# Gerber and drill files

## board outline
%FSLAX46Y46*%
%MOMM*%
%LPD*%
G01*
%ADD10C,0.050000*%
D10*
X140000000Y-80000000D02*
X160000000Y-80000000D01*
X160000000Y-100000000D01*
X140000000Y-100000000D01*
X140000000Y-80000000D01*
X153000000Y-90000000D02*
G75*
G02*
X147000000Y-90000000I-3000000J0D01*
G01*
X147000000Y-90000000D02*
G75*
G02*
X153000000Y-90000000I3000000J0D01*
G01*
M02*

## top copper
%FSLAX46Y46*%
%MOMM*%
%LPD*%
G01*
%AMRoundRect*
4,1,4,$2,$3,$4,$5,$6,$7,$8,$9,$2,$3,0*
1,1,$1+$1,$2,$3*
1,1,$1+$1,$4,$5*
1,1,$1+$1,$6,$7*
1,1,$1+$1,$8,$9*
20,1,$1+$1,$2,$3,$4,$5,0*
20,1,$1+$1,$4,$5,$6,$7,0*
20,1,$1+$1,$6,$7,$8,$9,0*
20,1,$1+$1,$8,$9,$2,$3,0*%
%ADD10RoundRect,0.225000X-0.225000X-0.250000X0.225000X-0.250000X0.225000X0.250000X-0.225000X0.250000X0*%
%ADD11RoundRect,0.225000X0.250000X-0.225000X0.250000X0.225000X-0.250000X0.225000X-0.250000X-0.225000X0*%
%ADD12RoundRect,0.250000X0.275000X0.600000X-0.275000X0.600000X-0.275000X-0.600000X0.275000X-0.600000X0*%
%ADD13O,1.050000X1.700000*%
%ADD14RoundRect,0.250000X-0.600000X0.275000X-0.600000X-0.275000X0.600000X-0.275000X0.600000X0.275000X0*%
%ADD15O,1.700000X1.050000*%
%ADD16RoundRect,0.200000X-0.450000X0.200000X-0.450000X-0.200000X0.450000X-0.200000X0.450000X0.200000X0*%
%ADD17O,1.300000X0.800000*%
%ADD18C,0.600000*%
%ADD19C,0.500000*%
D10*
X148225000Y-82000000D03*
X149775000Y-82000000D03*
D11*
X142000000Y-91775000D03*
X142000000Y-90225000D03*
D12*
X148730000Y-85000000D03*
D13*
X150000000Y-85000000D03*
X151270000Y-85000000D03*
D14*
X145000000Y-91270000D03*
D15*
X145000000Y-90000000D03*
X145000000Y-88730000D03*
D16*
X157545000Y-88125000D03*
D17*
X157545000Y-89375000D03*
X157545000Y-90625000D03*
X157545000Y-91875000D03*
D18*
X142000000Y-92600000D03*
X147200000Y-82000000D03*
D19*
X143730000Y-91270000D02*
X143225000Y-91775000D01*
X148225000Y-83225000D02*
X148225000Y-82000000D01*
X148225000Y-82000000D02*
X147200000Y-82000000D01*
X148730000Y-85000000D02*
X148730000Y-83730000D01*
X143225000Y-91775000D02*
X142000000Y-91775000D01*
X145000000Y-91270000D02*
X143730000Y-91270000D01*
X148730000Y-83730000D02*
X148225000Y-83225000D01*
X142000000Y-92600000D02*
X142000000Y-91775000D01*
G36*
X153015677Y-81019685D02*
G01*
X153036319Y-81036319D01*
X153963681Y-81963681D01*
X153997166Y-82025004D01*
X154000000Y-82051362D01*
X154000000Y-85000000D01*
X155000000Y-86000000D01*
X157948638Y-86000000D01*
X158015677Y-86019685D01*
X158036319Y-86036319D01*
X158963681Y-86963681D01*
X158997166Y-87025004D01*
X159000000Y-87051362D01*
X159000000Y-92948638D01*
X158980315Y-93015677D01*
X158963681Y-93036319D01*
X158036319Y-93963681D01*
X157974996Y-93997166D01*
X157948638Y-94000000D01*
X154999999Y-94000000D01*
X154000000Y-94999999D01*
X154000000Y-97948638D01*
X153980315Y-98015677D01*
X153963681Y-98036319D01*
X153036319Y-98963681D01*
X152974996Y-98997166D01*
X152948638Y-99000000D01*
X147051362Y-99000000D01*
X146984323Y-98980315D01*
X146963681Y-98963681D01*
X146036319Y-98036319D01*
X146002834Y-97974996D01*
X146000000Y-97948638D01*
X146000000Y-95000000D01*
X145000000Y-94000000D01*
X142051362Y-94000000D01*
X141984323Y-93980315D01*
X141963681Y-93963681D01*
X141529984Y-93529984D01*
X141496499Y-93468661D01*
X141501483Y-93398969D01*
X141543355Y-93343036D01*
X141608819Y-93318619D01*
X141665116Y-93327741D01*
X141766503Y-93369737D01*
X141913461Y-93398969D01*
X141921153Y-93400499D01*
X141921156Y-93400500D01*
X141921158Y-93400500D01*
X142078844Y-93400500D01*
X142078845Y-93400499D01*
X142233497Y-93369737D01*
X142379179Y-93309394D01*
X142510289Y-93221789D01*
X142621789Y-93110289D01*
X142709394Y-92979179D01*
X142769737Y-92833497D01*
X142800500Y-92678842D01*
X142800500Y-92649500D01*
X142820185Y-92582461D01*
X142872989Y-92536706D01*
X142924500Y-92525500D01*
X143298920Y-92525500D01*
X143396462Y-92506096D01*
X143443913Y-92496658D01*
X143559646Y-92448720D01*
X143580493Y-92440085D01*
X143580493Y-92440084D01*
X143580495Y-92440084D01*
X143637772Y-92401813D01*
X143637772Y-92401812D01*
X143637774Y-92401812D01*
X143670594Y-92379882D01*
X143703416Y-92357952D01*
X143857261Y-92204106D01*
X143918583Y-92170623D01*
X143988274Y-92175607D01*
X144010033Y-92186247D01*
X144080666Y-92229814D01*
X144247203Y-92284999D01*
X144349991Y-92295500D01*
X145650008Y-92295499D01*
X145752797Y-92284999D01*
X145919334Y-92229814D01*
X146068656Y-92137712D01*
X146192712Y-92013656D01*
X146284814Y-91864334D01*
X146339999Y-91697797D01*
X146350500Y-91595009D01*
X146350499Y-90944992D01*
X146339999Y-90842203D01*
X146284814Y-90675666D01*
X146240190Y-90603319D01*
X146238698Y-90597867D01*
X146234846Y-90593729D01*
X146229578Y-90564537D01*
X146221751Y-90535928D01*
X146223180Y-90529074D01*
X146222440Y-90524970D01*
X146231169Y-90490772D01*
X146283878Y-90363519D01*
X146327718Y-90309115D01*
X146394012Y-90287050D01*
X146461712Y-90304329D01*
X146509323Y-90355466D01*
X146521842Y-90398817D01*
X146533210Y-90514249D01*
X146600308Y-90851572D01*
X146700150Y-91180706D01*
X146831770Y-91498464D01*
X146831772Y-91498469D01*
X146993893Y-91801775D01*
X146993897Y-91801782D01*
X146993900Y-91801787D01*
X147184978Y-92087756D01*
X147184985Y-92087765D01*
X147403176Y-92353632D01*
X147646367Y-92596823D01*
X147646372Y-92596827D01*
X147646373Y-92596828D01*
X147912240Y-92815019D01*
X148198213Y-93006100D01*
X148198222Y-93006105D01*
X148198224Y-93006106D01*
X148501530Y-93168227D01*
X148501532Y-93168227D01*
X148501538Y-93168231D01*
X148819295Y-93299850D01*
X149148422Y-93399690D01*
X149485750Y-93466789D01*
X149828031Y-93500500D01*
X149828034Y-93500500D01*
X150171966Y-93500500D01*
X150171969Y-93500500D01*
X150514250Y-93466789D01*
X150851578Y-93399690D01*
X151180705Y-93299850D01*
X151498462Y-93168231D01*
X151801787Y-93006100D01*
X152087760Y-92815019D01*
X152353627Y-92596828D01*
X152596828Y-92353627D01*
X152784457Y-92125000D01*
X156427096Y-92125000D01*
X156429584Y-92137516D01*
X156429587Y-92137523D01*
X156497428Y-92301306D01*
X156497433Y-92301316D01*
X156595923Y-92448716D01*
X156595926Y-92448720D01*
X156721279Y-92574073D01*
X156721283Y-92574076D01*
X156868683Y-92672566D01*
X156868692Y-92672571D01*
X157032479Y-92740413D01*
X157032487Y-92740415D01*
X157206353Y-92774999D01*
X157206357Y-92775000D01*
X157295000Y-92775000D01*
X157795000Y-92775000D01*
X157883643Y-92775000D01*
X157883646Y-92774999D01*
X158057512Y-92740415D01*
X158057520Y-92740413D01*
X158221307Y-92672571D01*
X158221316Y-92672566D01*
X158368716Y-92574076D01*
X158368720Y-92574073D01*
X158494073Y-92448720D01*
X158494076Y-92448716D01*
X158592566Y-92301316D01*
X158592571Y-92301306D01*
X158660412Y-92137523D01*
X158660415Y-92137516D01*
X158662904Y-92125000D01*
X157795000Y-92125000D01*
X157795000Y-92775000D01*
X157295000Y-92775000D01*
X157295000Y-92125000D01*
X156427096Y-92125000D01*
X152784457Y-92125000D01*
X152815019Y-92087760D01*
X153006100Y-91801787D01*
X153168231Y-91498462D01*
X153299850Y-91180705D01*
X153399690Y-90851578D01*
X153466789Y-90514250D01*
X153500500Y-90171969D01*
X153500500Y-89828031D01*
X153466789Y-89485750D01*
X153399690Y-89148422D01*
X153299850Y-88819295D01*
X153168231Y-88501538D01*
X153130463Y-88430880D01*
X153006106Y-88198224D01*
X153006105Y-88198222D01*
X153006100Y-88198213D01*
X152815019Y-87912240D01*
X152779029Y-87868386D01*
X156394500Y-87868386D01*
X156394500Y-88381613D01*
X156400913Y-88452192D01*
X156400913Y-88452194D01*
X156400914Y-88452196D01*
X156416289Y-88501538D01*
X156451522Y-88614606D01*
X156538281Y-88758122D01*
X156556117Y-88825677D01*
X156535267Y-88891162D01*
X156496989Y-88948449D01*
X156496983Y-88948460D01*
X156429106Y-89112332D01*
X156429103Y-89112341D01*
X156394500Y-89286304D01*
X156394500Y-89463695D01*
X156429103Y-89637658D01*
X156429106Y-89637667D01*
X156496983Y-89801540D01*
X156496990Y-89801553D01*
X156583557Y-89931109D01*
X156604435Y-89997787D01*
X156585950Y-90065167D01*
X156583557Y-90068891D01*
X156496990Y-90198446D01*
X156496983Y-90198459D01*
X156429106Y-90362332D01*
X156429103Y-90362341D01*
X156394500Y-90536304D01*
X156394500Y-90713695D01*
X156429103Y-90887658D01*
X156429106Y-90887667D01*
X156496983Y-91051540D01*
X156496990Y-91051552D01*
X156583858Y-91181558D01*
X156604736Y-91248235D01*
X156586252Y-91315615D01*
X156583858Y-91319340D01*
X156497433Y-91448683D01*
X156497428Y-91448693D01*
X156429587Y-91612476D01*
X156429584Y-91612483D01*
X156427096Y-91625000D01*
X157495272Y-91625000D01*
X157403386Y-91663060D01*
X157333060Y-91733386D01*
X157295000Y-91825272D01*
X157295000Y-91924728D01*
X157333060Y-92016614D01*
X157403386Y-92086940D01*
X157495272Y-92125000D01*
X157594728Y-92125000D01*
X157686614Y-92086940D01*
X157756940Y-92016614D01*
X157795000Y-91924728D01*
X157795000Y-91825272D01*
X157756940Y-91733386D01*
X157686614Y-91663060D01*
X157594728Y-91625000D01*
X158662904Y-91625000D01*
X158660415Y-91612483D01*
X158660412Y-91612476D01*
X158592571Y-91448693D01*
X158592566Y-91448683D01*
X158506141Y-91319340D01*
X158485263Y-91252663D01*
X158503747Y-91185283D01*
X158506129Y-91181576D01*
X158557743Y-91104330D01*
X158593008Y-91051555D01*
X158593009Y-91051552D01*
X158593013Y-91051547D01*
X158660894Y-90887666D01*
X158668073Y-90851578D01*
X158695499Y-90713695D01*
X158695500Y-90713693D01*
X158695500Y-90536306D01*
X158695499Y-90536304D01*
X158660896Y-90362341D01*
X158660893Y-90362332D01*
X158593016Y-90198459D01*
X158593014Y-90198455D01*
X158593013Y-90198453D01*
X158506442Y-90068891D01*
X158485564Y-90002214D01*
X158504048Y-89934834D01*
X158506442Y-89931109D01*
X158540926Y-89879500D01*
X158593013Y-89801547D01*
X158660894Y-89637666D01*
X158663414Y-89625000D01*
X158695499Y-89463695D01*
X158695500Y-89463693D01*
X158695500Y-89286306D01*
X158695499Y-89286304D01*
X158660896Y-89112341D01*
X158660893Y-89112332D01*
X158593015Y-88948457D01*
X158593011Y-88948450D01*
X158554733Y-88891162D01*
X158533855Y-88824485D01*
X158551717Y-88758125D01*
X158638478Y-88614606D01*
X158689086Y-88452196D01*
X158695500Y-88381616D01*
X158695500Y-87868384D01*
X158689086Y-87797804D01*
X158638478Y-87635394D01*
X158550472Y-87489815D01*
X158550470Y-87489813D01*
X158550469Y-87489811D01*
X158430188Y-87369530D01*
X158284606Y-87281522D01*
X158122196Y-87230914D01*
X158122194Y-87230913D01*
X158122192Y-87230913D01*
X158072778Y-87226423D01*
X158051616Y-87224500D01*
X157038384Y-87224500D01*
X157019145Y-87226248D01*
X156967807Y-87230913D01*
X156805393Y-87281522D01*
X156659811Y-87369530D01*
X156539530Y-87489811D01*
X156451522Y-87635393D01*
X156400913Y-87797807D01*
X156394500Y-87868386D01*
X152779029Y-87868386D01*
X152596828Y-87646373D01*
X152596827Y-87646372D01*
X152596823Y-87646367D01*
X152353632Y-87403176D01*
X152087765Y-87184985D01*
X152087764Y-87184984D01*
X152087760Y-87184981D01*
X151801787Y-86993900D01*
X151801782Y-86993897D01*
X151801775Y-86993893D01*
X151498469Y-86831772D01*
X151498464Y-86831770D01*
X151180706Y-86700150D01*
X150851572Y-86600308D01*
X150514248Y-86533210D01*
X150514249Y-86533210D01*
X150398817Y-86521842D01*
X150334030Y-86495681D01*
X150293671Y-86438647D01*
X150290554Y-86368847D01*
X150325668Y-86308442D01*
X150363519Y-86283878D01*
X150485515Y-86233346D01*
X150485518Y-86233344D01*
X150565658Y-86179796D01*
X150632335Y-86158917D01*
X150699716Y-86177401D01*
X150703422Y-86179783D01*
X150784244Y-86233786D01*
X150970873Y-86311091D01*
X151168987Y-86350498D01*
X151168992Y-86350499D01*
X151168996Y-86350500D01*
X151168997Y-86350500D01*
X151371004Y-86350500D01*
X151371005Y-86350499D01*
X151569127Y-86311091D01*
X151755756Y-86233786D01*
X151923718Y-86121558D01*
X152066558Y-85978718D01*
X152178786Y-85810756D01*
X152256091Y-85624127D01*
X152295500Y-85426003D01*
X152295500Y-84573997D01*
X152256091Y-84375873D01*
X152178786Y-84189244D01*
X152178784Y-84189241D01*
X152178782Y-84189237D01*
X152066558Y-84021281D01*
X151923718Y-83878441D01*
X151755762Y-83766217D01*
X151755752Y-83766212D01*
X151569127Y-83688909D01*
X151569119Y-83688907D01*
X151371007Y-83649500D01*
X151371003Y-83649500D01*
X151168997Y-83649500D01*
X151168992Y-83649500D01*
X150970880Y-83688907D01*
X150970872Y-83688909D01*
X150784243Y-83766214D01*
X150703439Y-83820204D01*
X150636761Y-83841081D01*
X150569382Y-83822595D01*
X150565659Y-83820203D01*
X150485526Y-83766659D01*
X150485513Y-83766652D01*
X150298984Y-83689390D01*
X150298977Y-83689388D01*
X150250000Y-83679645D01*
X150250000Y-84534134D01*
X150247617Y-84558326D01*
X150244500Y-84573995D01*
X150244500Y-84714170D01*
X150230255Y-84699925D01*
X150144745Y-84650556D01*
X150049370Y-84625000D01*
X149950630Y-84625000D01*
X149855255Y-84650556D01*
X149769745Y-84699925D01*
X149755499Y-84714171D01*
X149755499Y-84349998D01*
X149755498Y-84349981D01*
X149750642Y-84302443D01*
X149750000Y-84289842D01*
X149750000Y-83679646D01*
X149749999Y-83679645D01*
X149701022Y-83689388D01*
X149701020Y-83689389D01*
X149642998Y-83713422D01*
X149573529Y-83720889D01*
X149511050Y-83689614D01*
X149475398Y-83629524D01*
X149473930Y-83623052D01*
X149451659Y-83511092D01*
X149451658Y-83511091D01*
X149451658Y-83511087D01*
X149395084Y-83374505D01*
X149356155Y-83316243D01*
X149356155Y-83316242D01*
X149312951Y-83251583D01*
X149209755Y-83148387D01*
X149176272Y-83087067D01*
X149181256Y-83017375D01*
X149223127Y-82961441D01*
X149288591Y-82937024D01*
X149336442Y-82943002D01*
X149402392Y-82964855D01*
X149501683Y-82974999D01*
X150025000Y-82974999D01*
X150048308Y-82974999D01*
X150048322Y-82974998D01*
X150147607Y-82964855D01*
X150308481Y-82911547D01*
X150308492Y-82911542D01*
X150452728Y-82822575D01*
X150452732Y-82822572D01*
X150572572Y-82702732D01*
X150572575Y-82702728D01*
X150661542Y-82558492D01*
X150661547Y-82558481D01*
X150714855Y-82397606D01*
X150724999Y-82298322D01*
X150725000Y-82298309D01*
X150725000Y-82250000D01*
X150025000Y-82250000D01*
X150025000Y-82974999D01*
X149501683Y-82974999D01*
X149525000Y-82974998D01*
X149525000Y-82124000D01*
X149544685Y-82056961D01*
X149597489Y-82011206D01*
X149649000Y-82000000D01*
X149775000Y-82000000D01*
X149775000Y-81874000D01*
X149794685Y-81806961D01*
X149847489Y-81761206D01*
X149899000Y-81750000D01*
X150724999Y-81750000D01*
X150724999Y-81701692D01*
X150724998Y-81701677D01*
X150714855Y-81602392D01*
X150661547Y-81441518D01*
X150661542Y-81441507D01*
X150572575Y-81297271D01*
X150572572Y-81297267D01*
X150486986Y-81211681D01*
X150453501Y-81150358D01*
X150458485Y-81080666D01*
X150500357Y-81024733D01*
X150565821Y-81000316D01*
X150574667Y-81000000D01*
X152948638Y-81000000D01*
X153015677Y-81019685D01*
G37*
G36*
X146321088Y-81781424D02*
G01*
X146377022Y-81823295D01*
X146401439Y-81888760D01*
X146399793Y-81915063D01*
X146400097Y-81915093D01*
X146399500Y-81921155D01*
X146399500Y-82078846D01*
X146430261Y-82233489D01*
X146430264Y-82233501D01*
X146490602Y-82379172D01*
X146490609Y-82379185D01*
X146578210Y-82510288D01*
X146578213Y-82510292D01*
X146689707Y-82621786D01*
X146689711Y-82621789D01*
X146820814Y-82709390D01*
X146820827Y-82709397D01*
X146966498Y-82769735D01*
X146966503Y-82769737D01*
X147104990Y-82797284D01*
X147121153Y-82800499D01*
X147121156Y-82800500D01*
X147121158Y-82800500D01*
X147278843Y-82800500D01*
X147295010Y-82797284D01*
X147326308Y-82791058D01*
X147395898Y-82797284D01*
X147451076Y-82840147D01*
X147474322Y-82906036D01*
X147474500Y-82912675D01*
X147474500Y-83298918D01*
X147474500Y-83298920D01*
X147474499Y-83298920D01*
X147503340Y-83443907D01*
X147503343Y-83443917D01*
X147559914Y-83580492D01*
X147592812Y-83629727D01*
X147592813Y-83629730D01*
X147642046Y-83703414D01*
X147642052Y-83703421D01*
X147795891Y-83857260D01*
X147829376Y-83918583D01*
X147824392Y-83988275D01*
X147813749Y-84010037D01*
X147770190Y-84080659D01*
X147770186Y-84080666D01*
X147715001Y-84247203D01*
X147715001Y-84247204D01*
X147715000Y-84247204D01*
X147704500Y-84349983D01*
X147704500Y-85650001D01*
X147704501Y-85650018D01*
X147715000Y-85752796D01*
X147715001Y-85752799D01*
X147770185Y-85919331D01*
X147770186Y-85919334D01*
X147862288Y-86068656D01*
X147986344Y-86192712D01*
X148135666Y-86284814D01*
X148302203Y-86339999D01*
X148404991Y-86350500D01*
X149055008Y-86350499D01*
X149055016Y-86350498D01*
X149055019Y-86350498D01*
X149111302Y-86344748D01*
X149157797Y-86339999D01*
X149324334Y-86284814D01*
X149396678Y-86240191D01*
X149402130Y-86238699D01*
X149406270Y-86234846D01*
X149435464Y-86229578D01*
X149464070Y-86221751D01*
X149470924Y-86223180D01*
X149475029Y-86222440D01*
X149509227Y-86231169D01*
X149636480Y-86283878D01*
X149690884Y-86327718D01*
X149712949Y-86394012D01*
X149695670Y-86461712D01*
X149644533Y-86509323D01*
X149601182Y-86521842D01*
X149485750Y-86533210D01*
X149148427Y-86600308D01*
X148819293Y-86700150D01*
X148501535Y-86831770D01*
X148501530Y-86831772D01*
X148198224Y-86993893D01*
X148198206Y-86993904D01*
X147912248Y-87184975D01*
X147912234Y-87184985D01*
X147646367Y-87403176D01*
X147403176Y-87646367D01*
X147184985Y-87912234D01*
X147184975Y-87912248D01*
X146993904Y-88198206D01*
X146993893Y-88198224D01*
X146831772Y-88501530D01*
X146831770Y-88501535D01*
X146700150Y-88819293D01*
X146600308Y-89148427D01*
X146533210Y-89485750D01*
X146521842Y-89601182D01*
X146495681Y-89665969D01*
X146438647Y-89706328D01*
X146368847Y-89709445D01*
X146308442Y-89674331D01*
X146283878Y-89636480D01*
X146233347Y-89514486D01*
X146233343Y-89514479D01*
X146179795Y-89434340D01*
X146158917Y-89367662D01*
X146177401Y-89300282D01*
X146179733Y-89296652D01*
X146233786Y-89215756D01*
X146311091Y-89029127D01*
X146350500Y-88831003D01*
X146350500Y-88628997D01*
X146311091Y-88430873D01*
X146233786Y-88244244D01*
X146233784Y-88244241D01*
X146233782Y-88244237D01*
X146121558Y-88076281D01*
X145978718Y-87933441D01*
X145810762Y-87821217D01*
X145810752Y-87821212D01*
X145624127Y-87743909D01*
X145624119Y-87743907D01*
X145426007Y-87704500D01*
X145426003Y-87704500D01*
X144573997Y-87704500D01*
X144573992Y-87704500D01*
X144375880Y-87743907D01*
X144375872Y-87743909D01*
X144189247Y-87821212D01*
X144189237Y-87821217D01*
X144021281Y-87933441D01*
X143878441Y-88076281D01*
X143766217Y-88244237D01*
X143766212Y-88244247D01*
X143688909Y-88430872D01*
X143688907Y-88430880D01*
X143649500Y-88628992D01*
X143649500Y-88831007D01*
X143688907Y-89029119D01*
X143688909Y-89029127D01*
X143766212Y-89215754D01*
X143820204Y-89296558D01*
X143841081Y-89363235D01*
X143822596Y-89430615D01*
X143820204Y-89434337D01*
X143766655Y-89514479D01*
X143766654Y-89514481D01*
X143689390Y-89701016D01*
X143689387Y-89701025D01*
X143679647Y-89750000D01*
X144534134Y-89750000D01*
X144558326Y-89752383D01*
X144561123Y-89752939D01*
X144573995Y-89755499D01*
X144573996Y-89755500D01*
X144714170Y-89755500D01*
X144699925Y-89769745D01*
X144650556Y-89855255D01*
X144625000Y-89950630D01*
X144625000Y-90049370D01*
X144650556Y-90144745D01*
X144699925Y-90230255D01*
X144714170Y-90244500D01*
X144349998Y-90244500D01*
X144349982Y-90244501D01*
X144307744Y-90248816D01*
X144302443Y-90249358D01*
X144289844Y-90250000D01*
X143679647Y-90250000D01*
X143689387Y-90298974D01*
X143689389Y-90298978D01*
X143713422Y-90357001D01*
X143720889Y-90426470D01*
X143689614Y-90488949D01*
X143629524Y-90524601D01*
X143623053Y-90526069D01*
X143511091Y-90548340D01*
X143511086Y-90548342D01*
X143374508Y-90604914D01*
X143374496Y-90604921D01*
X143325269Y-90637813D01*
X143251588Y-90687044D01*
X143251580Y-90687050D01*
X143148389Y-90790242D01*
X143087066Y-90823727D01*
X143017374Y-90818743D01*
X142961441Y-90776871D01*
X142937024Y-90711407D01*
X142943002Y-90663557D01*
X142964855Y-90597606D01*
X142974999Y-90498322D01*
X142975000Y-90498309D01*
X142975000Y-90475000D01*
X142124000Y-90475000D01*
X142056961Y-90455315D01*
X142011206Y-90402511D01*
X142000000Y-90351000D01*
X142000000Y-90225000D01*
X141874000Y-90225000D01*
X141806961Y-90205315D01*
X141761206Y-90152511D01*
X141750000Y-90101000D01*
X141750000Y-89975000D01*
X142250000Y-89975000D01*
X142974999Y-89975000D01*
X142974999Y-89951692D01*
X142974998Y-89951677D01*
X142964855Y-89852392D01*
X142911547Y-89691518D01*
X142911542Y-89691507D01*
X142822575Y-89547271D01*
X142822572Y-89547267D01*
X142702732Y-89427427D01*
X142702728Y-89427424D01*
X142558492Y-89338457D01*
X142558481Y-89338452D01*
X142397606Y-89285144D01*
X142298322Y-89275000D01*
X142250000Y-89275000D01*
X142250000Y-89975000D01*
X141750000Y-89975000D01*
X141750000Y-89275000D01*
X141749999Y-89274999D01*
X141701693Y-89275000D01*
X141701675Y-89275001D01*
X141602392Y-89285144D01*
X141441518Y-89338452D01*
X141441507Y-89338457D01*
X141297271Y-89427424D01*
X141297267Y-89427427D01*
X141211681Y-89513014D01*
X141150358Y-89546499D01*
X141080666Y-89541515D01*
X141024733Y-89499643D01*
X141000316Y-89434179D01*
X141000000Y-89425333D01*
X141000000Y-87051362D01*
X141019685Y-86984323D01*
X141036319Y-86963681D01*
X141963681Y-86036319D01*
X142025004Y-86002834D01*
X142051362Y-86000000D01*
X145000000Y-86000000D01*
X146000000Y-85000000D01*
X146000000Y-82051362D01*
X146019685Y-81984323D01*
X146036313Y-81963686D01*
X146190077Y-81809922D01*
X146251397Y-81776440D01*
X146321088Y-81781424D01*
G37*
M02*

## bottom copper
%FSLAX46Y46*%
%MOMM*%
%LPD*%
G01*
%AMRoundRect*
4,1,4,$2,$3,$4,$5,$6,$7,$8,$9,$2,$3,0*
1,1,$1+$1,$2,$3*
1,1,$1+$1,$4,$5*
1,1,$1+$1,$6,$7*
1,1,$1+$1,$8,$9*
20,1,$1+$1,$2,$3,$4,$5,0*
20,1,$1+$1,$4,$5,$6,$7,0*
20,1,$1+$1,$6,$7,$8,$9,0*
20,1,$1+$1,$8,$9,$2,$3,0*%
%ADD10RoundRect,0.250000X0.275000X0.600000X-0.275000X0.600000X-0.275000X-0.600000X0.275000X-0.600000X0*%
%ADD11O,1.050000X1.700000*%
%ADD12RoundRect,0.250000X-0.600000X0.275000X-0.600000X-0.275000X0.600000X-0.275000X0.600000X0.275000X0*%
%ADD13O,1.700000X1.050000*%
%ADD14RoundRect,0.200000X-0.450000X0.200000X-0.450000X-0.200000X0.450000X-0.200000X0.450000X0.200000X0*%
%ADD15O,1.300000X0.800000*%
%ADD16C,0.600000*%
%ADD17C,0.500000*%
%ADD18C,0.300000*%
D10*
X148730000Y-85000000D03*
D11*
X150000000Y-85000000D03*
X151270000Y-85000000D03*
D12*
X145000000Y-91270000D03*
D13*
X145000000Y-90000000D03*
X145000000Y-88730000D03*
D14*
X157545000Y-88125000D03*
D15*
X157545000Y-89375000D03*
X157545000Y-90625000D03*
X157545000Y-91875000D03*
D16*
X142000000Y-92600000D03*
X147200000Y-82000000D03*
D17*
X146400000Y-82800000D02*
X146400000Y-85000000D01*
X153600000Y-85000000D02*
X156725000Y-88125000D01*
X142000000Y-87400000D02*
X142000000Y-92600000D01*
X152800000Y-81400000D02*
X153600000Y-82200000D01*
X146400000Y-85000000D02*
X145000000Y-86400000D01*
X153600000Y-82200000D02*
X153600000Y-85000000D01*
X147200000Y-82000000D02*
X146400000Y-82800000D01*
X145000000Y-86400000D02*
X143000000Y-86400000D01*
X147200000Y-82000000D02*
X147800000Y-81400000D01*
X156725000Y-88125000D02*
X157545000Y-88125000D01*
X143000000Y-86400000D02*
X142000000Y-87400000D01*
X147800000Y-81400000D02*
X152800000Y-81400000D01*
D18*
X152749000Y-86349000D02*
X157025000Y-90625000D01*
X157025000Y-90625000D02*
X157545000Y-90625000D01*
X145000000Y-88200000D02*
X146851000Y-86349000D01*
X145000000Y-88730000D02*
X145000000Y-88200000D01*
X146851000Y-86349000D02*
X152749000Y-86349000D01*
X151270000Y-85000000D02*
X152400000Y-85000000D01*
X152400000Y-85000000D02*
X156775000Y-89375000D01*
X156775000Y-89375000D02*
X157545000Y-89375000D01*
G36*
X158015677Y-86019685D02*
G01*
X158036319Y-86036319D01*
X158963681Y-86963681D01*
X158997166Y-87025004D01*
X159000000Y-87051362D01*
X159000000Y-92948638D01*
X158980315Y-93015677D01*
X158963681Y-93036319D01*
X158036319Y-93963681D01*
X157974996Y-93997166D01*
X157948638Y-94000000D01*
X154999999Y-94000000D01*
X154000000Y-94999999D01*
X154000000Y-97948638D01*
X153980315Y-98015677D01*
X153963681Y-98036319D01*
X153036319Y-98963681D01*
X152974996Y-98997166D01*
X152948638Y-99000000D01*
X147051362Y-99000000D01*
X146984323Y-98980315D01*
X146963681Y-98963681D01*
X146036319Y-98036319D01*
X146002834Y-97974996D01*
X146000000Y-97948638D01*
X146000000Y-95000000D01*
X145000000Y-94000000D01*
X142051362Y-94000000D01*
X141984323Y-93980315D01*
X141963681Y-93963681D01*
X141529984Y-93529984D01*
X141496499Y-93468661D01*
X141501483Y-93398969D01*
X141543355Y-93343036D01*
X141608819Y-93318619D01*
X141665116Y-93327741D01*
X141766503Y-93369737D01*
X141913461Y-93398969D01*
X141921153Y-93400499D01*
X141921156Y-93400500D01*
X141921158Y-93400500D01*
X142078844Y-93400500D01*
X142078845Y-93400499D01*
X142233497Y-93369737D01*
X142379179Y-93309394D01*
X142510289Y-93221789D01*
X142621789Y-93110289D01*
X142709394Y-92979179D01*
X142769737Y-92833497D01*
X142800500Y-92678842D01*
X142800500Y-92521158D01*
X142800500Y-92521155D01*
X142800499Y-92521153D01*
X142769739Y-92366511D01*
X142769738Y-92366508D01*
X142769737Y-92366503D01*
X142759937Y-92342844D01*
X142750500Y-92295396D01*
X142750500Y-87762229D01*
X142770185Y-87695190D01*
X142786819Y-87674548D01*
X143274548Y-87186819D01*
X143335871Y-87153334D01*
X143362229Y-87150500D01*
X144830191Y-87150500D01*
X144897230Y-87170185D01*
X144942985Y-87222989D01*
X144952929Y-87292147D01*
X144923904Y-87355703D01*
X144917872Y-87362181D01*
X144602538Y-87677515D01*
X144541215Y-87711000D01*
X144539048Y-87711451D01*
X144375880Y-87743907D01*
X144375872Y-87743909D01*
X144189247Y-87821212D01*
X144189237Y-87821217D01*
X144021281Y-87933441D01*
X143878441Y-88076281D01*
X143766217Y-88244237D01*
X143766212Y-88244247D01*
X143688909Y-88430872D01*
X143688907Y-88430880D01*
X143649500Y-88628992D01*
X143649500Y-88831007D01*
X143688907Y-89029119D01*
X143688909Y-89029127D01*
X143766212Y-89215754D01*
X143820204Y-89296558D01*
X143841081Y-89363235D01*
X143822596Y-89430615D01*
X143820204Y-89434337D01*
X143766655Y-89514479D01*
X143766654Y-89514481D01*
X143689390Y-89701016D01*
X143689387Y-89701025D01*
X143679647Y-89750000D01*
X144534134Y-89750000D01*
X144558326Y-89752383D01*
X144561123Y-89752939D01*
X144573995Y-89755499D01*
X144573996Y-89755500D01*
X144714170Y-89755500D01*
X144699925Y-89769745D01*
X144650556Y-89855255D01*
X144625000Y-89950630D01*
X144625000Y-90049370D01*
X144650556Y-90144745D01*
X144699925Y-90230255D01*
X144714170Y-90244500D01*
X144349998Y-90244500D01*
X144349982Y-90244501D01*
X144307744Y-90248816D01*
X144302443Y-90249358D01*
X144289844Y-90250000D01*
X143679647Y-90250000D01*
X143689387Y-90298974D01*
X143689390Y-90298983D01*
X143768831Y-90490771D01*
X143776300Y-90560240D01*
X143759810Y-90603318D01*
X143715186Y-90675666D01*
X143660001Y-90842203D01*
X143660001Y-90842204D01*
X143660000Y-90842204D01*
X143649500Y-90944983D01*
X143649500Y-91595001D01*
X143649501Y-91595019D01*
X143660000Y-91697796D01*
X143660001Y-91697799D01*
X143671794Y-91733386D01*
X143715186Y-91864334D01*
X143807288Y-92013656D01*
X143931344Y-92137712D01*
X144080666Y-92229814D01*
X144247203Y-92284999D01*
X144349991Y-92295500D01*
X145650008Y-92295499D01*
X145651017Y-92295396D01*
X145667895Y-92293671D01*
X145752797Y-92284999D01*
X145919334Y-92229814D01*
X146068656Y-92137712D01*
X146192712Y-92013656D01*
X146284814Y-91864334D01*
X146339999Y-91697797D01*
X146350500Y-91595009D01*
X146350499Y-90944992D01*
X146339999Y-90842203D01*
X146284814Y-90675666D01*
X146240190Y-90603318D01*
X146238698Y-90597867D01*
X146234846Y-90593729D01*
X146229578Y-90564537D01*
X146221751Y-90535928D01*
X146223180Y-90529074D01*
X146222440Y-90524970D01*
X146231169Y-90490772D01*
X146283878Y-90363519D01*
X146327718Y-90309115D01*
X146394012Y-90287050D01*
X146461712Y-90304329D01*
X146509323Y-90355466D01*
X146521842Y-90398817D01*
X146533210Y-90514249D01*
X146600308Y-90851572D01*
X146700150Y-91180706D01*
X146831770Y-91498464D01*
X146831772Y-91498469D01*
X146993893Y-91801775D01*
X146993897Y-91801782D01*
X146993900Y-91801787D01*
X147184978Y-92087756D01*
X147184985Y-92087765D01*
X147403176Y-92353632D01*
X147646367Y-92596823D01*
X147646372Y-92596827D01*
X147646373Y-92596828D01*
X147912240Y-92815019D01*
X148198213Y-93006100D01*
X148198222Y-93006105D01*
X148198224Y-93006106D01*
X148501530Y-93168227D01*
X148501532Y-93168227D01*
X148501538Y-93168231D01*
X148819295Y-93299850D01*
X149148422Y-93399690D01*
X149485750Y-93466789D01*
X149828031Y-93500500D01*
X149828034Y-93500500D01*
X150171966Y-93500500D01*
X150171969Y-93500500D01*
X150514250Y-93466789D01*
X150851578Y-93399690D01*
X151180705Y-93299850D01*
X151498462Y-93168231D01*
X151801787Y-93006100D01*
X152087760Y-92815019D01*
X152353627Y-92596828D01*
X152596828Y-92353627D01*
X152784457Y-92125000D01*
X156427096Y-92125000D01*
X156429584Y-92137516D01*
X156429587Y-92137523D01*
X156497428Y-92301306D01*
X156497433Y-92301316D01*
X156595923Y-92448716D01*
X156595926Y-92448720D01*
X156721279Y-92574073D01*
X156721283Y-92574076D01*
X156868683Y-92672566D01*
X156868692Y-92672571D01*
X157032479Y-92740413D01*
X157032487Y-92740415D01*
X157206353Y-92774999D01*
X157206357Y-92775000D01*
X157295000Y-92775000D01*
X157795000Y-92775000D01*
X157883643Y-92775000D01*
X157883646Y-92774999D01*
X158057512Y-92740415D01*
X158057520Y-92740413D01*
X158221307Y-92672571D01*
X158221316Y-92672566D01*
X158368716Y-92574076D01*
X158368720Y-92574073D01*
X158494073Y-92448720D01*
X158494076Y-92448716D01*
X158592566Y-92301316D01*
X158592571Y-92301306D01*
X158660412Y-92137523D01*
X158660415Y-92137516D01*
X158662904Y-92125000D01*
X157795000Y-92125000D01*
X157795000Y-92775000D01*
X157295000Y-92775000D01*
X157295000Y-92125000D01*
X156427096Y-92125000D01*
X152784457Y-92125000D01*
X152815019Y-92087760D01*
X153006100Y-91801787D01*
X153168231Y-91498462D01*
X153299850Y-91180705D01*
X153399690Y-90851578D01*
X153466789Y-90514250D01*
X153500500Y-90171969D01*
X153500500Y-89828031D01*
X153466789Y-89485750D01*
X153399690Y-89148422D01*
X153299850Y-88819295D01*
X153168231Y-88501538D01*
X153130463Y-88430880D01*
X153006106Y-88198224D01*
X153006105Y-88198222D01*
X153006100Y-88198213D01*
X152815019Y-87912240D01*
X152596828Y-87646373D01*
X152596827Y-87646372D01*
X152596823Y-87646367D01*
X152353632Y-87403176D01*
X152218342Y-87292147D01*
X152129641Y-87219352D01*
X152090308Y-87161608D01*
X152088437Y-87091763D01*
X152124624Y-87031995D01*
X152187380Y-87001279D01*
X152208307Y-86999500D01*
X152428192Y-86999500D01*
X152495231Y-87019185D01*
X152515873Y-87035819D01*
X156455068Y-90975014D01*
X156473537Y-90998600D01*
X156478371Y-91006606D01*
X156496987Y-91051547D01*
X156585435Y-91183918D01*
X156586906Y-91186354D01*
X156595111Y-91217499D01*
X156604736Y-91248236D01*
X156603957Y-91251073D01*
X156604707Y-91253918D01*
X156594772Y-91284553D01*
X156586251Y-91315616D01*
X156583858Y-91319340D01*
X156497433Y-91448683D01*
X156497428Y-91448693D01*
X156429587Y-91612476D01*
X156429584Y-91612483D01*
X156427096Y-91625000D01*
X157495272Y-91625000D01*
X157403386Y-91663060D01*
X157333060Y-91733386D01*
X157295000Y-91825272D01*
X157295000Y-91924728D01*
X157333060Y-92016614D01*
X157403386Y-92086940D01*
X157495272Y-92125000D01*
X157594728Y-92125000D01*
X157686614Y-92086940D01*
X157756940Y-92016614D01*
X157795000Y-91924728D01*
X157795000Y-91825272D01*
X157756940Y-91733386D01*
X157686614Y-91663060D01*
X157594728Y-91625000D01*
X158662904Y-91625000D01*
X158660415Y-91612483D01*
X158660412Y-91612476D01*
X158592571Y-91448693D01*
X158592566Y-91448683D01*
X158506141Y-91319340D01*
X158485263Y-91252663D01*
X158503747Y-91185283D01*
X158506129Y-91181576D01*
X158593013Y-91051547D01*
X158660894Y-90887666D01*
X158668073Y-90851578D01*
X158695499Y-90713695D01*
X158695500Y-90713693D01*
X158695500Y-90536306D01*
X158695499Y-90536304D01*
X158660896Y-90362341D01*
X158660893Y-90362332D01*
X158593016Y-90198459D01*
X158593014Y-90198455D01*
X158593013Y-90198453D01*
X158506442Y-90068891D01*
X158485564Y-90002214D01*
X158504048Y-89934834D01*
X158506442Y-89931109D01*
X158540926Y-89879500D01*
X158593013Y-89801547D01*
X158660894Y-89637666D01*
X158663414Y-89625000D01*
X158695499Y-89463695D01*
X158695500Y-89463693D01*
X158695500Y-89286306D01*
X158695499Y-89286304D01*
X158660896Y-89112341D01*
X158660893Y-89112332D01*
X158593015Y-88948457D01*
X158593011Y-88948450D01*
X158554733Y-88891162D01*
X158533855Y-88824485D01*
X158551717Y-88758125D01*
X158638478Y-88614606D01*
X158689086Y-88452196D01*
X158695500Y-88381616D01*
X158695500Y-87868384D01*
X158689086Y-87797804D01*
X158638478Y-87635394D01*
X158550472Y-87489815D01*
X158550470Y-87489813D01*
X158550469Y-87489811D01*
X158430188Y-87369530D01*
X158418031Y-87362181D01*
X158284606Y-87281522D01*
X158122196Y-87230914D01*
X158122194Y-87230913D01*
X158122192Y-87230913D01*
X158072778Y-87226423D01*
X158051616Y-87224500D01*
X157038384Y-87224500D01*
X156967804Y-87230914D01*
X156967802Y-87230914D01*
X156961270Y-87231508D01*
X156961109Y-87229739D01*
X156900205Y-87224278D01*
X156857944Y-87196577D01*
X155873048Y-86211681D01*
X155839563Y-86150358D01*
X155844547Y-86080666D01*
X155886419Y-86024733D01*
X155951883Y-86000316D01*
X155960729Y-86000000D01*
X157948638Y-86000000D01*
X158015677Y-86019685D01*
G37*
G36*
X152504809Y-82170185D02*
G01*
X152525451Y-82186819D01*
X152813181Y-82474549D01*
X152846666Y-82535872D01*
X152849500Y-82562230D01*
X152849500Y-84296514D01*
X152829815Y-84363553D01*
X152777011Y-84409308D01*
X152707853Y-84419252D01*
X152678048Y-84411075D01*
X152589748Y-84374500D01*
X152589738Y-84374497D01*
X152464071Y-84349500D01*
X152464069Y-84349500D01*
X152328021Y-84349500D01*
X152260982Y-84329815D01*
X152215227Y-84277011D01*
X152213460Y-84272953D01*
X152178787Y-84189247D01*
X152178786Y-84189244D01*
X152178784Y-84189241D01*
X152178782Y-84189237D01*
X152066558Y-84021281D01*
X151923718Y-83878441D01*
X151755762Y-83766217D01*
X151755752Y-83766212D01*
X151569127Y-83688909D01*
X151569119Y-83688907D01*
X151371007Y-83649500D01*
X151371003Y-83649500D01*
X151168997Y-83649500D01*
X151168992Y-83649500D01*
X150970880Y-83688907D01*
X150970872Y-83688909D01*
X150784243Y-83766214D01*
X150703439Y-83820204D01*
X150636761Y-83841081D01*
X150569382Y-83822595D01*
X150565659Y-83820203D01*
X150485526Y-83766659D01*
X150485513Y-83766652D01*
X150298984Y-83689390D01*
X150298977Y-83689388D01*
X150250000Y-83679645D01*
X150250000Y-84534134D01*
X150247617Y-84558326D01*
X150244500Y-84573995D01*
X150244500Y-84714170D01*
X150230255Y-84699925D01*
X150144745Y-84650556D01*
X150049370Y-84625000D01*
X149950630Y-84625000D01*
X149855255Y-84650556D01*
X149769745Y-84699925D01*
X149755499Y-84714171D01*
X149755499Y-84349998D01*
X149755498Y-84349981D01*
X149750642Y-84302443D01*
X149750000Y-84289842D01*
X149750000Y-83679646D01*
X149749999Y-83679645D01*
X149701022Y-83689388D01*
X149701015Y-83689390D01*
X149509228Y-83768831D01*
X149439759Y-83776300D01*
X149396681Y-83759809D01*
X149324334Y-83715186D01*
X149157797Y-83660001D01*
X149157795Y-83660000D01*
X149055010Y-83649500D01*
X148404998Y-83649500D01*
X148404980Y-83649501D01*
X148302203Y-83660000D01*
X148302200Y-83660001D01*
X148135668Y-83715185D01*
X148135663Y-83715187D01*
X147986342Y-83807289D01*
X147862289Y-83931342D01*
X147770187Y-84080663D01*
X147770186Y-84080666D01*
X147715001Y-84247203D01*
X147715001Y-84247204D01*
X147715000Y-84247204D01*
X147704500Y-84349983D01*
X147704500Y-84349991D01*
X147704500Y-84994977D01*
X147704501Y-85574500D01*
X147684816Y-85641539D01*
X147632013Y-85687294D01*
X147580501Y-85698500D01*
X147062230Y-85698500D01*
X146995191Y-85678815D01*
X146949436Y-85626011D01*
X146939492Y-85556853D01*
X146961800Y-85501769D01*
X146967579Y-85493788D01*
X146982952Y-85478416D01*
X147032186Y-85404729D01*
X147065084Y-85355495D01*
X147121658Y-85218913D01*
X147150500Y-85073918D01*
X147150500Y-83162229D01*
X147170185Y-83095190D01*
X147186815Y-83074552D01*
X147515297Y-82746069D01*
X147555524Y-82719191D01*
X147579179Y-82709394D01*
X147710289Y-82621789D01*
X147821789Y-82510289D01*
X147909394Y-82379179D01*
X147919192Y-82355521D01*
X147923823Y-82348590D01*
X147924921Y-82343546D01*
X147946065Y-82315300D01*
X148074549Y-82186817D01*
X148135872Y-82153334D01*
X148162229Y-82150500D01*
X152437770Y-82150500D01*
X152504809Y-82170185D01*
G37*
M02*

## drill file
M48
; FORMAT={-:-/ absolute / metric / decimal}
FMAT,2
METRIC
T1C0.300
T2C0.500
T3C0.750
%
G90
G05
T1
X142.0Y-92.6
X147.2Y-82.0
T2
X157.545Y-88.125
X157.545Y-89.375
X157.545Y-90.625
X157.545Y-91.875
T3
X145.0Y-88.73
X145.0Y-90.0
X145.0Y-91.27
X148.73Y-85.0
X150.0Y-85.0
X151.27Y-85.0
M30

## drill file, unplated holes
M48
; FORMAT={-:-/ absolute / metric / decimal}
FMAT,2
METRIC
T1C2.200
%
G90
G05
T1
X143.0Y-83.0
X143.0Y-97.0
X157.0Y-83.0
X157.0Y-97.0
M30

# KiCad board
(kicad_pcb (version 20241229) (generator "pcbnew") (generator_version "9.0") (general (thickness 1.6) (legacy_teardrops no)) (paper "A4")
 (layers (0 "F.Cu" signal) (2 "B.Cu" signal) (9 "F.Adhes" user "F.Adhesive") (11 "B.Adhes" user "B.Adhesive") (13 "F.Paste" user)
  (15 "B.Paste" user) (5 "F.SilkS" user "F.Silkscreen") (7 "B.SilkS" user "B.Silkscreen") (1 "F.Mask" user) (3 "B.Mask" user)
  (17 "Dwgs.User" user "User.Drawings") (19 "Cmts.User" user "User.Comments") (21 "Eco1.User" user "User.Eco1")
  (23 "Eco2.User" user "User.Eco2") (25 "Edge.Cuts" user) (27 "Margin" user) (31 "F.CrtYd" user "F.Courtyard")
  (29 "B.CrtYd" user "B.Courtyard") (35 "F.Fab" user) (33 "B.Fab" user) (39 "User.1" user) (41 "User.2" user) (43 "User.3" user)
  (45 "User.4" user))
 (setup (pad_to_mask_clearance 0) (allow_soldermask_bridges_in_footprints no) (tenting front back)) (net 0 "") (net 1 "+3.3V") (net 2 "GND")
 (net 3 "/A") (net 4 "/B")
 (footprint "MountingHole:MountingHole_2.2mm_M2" (layer "F.Cu") (at 157 83)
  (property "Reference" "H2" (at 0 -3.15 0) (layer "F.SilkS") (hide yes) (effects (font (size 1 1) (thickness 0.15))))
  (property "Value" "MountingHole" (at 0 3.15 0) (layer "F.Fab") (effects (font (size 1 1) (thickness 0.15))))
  (pad "" np_thru_hole circle (at 0 0) (size 2.2 2.2) (drill 2.2) (layers "*.Cu" "*.Mask")))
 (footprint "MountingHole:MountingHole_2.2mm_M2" (layer "F.Cu") (at 143 83)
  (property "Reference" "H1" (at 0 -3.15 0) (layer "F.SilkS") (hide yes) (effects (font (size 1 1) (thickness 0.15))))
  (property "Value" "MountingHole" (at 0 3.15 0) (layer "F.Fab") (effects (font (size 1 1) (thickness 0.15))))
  (pad "" np_thru_hole circle (at 0 0) (size 2.2 2.2) (drill 2.2) (layers "*.Cu" "*.Mask")))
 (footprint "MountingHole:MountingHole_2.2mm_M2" (layer "F.Cu") (at 157 97)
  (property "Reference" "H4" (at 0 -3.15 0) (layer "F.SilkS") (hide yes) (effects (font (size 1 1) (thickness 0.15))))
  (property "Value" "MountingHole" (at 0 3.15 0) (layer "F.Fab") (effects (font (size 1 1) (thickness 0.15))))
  (pad "" np_thru_hole circle (at 0 0) (size 2.2 2.2) (drill 2.2) (layers "*.Cu" "*.Mask")))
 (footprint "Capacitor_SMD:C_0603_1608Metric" (layer "F.Cu") (at 149 82)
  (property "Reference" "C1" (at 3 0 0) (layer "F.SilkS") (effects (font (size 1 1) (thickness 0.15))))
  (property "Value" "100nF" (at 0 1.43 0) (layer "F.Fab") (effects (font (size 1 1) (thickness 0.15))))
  (pad "1" smd roundrect (at -0.775 0) (size 0.9 0.95) (layers "F.Cu" "F.Mask" "F.Paste") (roundrect_rratio 0.25) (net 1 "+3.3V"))
  (pad "2" smd roundrect (at 0.775 0) (size 0.9 0.95) (layers "F.Cu" "F.Mask" "F.Paste") (roundrect_rratio 0.25) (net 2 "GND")))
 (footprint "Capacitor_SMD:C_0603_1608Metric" (layer "F.Cu") (at 142 91 90)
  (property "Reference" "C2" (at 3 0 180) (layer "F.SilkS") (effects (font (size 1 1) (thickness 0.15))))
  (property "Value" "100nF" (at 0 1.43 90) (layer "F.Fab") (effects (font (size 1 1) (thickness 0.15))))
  (pad "1" smd roundrect (at -0.775 0 90) (size 0.9 0.95) (layers "F.Cu" "F.Mask" "F.Paste") (roundrect_rratio 0.25) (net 1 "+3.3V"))
  (pad "2" smd roundrect (at 0.775 0 90) (size 0.9 0.95) (layers "F.Cu" "F.Mask" "F.Paste") (roundrect_rratio 0.25) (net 2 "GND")))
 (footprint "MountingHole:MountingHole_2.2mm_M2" (layer "F.Cu") (at 143 97)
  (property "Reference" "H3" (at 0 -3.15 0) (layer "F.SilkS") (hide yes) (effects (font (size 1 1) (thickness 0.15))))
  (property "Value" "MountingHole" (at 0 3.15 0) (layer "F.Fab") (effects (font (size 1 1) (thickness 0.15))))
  (pad "" np_thru_hole circle (at 0 0) (size 2.2 2.2) (drill 2.2) (layers "*.Cu" "*.Mask")))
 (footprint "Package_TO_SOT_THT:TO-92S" (layer "F.Cu") (at 148.73 85)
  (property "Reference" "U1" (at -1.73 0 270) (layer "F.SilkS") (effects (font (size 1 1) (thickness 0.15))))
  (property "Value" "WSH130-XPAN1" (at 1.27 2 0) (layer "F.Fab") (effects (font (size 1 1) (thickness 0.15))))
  (pad "1" thru_hole roundrect (at 0 0 180) (size 1.05 1.7) (drill 0.75) (layers "*.Cu" "*.Mask") (remove_unused_layers no)
   (roundrect_rratio 0.2380952381) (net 1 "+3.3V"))
  (pad "2" thru_hole oval (at 1.27 0 180) (size 1.05 1.7) (drill 0.75) (layers "*.Cu" "*.Mask") (remove_unused_layers no) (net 2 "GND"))
  (pad "3" thru_hole oval (at 2.54 0 180) (size 1.05 1.7) (drill 0.75) (layers "*.Cu" "*.Mask") (remove_unused_layers no) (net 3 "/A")))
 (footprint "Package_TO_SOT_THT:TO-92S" (layer "F.Cu") (at 145 91.27 90)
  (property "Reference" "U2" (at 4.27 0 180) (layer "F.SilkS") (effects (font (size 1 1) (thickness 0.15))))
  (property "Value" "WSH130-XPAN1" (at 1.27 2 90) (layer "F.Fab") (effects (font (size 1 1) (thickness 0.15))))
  (pad "1" thru_hole roundrect (at 0 0 270) (size 1.05 1.7) (drill 0.75) (layers "*.Cu" "*.Mask") (remove_unused_layers no)
   (roundrect_rratio 0.2380952381) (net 1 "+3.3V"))
  (pad "2" thru_hole oval (at 1.27 0 270) (size 1.05 1.7) (drill 0.75) (layers "*.Cu" "*.Mask") (remove_unused_layers no) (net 2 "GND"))
  (pad "3" thru_hole oval (at 2.54 0 270) (size 1.05 1.7) (drill 0.75) (layers "*.Cu" "*.Mask") (remove_unused_layers no) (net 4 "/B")))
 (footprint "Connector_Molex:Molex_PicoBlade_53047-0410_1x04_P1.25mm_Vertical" (layer "F.Cu") (at 157.545 88.125 -90)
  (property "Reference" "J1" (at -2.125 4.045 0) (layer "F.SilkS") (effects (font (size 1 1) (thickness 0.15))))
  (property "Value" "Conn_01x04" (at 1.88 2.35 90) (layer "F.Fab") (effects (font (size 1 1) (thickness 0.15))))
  (pad "1" thru_hole roundrect (at 0 0 270) (size 0.8 1.3) (drill 0.5) (layers "*.Cu" "*.Mask") (remove_unused_layers no)
   (roundrect_rratio 0.25) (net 1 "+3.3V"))
  (pad "2" thru_hole oval (at 1.25 0 270) (size 0.8 1.3) (drill 0.5) (layers "*.Cu" "*.Mask") (remove_unused_layers no) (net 3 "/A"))
  (pad "3" thru_hole oval (at 2.5 0 270) (size 0.8 1.3) (drill 0.5) (layers "*.Cu" "*.Mask") (remove_unused_layers no) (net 4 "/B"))
  (pad "4" thru_hole oval (at 3.75 0 270) (size 0.8 1.3) (drill 0.5) (layers "*.Cu" "*.Mask") (remove_unused_layers no) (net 2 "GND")))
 (gr_rect (start 140 80) (end 160 100) (stroke (width 0.05) (type default)) (fill no) (layer "Edge.Cuts"))
 (gr_circle (center 150 90) (end 153 90) (stroke (width 0.05) (type default)) (fill no) (layer "Edge.Cuts"))
 (segment (start 143.73 91.27) (end 143.225 91.775) (width 0.5) (layer "F.Cu") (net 1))
 (segment (start 148.225 83.225) (end 148.225 82) (width 0.5) (layer "F.Cu") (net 1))
 (segment (start 148.225 82) (end 147.2 82) (width 0.5) (layer "F.Cu") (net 1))
 (segment (start 148.73 85) (end 148.73 83.73) (width 0.5) (layer "F.Cu") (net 1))
 (segment (start 143.225 91.775) (end 142 91.775) (width 0.5) (layer "F.Cu") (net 1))
 (segment (start 145 91.27) (end 143.73 91.27) (width 0.5) (layer "F.Cu") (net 1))
 (segment (start 148.73 83.73) (end 148.225 83.225) (width 0.5) (layer "F.Cu") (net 1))
 (segment (start 142 92.6) (end 142 91.775) (width 0.5) (layer "F.Cu") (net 1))
 (via (at 142 92.6) (size 0.6) (drill 0.3) (layers "F.Cu" "B.Cu") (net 1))
 (via (at 147.2 82) (size 0.6) (drill 0.3) (layers "F.Cu" "B.Cu") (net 1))
 (segment (start 146.4 82.8) (end 146.4 85) (width 0.5) (layer "B.Cu") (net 1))
 (segment (start 153.6 85) (end 156.725 88.125) (width 0.5) (layer "B.Cu") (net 1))
 (segment (start 142 87.4) (end 142 92.6) (width 0.5) (layer "B.Cu") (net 1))
 (segment (start 152.8 81.4) (end 153.6 82.2) (width 0.5) (layer "B.Cu") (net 1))
 (segment (start 146.4 85) (end 145 86.4) (width 0.5) (layer "B.Cu") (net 1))
 (segment (start 153.6 82.2) (end 153.6 85) (width 0.5) (layer "B.Cu") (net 1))
 (segment (start 147.2 82) (end 146.4 82.8) (width 0.5) (layer "B.Cu") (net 1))
 (segment (start 145 86.4) (end 143 86.4) (width 0.5) (layer "B.Cu") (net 1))
 (segment (start 147.2 82) (end 147.8 81.4) (width 0.5) (layer "B.Cu") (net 1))
 (segment (start 156.725 88.125) (end 157.545 88.125) (width 0.5) (layer "B.Cu") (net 1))
 (segment (start 143 86.4) (end 142 87.4) (width 0.5) (layer "B.Cu") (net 1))
 (segment (start 147.8 81.4) (end 152.8 81.4) (width 0.5) (layer "B.Cu") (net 1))
 (segment (start 152.749 86.349) (end 157.025 90.625) (width 0.3) (layer "B.Cu") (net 4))
 (segment (start 157.025 90.625) (end 157.545 90.625) (width 0.3) (layer "B.Cu") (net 4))
 (segment (start 145 88.2) (end 146.851 86.349) (width 0.3) (layer "B.Cu") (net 4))
 (segment (start 145 88.73) (end 145 88.2) (width 0.3) (layer "B.Cu") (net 4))
 (segment (start 146.851 86.349) (end 152.749 86.349) (width 0.3) (layer "B.Cu") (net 4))
 (segment (start 151.27 85) (end 152.4 85) (width 0.3) (layer "B.Cu") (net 3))
 (segment (start 152.4 85) (end 156.775 89.375) (width 0.3) (layer "B.Cu") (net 3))
 (segment (start 156.775 89.375) (end 157.545 89.375) (width 0.3) (layer "B.Cu") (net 3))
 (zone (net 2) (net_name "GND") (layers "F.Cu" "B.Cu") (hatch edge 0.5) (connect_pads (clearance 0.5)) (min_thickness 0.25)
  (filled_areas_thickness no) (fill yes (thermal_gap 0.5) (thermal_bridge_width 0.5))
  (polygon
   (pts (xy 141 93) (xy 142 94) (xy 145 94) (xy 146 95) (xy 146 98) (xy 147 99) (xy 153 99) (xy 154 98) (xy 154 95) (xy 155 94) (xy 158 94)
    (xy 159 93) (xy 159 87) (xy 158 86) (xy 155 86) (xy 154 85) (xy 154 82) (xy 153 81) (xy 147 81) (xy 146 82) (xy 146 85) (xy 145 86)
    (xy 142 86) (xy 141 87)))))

